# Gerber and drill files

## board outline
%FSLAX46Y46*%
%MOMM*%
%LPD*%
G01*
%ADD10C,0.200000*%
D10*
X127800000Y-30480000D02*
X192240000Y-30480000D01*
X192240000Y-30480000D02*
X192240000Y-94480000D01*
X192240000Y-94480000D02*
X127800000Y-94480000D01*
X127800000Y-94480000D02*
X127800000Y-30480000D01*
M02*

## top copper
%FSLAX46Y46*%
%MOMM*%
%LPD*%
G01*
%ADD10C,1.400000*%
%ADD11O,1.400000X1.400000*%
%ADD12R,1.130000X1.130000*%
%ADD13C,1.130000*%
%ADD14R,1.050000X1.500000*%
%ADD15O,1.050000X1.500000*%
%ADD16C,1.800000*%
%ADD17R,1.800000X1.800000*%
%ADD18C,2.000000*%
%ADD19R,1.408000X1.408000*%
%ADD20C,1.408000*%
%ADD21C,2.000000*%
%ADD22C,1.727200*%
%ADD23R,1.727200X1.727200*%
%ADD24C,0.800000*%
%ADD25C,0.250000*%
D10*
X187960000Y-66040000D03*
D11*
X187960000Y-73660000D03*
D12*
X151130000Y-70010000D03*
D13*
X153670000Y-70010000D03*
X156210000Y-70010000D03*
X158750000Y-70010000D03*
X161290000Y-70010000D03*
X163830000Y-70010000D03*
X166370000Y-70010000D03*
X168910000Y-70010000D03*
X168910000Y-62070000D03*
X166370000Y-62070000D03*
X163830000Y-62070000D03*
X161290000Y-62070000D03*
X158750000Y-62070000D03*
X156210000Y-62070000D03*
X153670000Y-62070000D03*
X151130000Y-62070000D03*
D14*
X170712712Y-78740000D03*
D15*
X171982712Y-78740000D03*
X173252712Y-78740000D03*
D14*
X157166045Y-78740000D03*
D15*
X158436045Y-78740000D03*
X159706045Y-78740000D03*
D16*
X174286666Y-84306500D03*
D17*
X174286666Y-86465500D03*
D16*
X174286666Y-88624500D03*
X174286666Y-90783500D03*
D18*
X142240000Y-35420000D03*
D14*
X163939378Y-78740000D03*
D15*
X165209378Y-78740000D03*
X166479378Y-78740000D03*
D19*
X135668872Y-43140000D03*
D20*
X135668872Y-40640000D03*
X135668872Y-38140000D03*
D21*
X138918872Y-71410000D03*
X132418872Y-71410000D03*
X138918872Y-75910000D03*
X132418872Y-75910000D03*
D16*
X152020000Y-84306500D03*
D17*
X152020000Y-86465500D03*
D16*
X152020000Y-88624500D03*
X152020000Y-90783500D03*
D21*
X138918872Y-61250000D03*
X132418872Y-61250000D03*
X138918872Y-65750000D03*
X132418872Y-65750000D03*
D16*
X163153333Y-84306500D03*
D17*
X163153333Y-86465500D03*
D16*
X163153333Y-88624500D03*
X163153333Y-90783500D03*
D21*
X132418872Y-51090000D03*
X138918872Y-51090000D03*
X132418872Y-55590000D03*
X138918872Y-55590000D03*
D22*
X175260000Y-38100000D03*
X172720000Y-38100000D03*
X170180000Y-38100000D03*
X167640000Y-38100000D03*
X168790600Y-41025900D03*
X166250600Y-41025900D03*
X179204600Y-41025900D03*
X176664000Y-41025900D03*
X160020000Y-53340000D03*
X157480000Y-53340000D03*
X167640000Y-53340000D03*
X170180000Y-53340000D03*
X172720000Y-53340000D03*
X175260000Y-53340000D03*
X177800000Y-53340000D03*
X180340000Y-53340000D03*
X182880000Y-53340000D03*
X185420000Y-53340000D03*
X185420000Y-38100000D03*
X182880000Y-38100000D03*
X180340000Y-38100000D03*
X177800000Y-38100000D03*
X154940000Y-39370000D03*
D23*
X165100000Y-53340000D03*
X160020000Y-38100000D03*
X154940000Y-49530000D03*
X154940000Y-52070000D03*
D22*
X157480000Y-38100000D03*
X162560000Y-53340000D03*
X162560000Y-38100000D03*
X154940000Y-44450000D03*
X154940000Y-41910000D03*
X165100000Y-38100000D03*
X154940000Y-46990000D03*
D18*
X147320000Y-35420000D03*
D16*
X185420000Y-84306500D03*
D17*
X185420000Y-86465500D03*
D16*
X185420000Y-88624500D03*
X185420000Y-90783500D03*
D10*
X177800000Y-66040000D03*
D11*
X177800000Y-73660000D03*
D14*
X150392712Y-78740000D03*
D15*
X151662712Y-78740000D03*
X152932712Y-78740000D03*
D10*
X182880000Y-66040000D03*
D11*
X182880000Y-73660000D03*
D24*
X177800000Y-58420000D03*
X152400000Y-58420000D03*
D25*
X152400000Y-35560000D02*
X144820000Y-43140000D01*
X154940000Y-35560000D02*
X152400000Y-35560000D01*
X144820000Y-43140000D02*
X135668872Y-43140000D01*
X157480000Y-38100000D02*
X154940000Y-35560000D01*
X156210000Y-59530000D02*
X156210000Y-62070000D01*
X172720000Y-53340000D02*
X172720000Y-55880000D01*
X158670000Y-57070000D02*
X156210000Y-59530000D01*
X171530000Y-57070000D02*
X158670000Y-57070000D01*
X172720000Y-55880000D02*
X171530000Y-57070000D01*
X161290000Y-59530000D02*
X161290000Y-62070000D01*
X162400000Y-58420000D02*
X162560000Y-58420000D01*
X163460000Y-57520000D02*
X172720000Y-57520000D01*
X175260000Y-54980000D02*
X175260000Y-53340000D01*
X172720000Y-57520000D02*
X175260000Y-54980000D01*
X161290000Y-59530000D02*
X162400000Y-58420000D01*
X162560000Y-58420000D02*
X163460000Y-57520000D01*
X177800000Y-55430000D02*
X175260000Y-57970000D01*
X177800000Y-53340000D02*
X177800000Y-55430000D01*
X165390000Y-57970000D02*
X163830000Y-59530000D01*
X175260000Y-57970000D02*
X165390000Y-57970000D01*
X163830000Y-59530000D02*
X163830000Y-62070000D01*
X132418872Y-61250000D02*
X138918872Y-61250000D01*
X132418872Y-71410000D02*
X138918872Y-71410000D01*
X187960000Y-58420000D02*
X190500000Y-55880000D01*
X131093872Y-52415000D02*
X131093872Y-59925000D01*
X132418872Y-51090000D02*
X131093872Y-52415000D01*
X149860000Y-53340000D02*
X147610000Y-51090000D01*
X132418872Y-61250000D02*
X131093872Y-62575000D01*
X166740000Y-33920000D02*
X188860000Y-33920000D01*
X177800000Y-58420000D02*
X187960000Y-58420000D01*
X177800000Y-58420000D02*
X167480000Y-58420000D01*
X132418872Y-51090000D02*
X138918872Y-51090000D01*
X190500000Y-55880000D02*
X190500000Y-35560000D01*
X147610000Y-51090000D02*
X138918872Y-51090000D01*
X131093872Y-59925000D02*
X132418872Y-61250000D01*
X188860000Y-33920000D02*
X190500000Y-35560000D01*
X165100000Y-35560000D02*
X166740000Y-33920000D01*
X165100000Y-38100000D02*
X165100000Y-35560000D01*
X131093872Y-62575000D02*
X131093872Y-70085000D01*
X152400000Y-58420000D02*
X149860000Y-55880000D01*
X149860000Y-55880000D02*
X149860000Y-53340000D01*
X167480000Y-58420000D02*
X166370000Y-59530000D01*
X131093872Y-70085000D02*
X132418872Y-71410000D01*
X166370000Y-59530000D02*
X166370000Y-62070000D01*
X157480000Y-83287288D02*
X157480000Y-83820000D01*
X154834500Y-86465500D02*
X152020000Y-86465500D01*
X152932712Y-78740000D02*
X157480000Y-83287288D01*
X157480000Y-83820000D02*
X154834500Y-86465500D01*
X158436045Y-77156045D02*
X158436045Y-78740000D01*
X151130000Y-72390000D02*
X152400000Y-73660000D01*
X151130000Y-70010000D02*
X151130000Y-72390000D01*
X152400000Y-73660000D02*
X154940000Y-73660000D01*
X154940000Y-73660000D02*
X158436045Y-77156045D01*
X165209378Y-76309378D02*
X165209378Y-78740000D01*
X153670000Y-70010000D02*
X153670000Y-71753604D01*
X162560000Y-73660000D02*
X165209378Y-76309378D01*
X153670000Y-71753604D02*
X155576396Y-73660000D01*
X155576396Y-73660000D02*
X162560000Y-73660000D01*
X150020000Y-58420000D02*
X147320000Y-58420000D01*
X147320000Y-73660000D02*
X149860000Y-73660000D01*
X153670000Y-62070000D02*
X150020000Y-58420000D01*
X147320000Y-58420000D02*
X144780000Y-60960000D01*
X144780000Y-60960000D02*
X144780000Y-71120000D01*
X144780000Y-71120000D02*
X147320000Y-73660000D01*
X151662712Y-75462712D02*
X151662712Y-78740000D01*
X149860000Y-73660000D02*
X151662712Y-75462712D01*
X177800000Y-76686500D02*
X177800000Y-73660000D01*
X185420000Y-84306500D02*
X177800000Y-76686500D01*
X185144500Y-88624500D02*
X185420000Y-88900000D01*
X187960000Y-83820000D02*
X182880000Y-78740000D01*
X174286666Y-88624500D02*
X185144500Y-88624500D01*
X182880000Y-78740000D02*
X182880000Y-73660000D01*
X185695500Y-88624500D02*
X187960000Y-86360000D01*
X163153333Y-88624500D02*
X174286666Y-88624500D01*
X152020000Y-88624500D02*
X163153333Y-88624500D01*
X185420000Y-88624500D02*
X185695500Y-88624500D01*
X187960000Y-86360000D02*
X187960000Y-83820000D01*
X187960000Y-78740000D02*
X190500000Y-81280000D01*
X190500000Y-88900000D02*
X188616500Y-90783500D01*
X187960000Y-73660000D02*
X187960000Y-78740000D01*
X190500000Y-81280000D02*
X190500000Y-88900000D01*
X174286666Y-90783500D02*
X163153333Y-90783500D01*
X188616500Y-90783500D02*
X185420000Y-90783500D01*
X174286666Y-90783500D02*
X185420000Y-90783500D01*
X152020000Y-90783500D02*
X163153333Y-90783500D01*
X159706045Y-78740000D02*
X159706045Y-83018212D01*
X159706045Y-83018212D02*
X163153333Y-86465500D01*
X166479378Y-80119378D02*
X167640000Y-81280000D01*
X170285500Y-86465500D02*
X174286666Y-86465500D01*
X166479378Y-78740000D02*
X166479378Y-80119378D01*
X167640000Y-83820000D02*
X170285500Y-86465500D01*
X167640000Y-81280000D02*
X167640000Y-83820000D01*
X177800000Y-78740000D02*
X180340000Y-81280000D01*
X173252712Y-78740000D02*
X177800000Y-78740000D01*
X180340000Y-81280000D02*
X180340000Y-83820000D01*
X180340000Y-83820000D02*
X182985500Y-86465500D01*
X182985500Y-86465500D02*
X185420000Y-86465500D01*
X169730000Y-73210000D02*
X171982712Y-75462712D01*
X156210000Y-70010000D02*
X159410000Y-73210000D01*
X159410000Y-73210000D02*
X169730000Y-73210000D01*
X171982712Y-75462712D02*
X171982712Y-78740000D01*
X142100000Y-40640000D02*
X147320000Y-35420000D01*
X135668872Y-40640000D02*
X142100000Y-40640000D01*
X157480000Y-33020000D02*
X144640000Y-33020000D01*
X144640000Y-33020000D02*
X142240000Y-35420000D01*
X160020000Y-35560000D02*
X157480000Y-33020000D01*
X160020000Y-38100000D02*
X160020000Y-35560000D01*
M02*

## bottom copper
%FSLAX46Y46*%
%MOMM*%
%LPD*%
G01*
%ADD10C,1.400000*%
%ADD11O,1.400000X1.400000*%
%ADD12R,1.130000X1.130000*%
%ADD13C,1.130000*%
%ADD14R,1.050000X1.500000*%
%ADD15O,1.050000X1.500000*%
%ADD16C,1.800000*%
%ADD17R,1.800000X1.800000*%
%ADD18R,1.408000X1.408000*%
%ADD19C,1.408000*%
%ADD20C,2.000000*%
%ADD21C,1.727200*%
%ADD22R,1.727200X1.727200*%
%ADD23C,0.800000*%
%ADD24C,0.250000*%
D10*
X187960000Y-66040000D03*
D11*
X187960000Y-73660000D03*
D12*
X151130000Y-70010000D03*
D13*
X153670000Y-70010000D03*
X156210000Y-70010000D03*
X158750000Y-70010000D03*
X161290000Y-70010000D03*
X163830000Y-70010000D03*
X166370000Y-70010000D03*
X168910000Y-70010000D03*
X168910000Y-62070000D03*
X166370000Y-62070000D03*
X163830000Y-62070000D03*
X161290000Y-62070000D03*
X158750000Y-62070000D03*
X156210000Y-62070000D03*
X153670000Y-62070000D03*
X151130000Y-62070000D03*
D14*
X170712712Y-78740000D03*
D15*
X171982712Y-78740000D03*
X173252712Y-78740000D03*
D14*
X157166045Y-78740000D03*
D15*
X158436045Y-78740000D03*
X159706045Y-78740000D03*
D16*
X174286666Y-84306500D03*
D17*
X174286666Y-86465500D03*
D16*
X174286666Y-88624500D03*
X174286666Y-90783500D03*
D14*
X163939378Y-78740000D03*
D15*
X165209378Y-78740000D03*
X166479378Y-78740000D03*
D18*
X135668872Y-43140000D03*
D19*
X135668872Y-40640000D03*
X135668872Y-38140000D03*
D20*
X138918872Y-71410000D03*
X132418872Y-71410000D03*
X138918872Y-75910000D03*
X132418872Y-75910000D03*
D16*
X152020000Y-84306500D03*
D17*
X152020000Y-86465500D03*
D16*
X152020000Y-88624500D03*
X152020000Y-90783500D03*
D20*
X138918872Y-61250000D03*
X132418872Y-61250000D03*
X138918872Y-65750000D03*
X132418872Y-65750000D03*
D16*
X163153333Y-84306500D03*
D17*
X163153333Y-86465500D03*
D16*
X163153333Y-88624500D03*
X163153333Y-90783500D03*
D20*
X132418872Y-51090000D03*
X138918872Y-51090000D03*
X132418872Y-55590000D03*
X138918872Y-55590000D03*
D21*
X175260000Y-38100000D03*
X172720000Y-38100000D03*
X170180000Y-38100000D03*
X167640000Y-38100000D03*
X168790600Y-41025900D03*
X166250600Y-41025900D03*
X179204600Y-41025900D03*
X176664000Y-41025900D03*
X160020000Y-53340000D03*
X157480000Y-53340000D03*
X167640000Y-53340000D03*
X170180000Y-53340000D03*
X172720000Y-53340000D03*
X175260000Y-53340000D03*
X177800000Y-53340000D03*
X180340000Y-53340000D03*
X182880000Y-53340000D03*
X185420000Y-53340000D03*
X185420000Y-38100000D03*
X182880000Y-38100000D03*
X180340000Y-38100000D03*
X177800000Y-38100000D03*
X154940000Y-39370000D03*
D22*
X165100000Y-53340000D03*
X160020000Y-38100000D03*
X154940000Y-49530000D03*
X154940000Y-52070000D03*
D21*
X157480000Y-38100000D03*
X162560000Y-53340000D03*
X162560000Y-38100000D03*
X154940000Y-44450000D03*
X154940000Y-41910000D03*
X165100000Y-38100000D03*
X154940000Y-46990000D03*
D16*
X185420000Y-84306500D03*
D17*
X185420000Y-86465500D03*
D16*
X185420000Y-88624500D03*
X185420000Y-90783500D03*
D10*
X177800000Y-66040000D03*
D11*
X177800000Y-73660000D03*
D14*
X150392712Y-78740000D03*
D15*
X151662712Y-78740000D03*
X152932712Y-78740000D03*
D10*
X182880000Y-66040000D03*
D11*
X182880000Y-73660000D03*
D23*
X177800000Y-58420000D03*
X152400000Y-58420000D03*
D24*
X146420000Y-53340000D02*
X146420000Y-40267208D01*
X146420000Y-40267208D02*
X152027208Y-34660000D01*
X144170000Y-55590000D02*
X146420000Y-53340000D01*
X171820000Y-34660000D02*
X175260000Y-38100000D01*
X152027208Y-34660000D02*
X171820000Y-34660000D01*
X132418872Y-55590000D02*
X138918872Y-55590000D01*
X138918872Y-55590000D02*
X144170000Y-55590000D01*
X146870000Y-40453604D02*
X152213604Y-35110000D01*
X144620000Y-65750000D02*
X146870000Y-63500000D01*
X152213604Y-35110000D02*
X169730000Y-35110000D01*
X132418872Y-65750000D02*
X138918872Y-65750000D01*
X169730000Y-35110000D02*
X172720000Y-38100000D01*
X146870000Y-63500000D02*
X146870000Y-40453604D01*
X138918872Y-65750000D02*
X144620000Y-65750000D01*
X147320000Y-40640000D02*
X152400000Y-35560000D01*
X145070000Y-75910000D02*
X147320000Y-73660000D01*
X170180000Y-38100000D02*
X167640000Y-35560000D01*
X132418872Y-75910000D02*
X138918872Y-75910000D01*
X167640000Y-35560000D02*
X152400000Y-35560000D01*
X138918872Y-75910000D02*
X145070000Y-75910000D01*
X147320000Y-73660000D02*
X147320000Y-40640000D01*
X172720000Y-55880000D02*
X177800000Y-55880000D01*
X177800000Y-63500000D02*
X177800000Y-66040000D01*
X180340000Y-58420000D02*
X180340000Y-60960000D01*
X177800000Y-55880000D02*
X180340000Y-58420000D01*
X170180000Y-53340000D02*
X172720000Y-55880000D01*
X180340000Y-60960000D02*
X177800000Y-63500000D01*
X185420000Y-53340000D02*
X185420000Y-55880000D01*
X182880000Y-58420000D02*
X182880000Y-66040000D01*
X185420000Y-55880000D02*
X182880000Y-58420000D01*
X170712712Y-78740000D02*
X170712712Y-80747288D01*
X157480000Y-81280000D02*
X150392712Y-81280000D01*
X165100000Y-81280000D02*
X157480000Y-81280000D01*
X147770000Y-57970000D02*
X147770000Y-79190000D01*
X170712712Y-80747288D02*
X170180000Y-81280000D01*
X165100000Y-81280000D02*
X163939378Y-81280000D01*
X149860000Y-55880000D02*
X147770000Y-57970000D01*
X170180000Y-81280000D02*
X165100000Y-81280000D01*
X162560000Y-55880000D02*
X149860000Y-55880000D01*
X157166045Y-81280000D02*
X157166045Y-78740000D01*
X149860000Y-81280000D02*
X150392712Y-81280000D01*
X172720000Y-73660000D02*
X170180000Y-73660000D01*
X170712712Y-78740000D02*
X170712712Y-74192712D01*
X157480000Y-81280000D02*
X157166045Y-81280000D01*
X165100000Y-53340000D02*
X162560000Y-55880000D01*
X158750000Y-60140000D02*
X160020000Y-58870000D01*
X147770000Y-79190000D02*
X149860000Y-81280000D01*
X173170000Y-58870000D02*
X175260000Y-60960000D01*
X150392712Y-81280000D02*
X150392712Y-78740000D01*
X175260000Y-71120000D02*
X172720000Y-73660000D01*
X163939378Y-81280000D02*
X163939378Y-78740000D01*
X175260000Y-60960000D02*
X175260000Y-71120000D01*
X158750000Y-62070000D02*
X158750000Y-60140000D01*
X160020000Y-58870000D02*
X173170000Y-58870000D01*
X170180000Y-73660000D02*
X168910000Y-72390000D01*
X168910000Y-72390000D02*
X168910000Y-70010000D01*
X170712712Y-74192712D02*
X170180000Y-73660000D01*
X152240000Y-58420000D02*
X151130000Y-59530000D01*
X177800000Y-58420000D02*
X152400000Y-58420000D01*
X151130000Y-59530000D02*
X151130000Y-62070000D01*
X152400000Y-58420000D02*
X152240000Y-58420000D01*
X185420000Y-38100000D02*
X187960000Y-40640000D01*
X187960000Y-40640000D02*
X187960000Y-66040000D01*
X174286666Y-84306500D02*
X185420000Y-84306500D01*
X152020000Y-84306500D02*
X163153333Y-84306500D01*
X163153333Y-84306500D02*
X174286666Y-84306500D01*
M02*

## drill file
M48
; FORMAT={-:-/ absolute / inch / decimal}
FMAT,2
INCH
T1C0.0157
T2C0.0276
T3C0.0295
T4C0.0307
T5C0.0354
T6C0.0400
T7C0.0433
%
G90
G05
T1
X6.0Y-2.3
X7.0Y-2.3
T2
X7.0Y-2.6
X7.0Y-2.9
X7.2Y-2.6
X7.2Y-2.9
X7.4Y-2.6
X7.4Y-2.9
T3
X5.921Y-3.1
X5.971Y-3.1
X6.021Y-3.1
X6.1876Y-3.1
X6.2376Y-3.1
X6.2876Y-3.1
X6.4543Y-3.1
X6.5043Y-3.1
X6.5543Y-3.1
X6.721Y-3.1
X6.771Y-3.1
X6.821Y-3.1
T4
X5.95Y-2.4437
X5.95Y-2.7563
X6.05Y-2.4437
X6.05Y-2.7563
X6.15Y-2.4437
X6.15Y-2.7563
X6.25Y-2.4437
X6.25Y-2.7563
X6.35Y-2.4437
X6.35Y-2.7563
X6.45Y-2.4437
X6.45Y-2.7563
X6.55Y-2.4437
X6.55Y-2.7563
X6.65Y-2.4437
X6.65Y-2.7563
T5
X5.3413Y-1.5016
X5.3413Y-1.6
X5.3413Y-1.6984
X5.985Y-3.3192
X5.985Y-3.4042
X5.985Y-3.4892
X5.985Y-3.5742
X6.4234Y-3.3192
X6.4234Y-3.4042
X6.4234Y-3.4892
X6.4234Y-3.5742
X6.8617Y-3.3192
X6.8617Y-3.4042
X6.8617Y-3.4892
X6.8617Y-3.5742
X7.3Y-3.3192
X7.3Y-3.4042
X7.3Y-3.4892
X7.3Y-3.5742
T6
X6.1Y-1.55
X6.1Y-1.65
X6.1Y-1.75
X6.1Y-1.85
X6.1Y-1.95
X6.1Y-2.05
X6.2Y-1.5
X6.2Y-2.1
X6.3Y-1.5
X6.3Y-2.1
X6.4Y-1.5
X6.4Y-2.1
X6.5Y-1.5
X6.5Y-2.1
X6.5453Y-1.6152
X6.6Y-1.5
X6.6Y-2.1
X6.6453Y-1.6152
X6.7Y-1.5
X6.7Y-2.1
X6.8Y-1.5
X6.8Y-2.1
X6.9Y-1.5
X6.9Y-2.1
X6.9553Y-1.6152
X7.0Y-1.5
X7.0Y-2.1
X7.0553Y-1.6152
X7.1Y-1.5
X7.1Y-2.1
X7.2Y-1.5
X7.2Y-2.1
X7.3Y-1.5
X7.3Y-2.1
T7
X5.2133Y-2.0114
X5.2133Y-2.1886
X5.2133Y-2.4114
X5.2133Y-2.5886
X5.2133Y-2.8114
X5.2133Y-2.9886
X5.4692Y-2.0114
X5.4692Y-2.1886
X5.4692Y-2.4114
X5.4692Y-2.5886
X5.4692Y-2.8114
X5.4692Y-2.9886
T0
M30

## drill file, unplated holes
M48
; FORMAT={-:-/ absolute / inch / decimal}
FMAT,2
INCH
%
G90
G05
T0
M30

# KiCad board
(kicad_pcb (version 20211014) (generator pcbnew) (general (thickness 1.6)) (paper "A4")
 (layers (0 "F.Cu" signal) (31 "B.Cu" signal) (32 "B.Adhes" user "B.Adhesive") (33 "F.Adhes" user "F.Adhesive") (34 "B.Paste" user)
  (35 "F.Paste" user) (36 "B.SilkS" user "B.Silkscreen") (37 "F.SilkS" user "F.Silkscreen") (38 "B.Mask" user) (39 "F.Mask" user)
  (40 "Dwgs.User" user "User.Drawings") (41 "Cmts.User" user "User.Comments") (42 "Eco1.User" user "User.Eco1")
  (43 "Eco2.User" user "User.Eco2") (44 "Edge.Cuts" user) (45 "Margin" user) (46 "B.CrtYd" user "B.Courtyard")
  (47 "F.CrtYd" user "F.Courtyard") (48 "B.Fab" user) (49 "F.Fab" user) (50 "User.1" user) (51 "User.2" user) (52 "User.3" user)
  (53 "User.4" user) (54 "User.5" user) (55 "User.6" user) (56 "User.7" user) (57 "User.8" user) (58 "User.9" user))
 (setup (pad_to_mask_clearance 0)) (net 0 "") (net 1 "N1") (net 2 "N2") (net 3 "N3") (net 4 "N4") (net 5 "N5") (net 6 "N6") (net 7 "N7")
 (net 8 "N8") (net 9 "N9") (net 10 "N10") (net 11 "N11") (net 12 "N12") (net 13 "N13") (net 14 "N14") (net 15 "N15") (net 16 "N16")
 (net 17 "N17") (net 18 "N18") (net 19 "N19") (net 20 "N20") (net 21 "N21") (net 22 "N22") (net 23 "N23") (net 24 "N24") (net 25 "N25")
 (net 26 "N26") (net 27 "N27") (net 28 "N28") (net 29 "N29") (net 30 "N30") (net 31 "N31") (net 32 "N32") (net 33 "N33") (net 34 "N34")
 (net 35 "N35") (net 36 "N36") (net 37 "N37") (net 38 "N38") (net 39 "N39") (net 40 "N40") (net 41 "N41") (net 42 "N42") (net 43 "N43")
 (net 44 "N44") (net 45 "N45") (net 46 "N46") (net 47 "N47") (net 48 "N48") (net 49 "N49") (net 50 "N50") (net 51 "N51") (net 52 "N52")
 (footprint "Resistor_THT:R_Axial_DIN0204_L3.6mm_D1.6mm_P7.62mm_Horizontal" (layer "F.Cu") (at 187.96 66.04 -90)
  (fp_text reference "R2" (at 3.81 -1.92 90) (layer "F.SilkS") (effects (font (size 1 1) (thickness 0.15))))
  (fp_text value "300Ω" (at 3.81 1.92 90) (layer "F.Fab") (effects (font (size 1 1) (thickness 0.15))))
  (pad "1" thru_hole circle (at 0 0 270) (size 1.4 1.4) (drill 0.7) (layers *.Cu *.Mask) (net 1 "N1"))
  (pad "2" thru_hole oval (at 7.62 0 270) (size 1.4 1.4) (drill 0.7) (layers *.Cu *.Mask) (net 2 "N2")))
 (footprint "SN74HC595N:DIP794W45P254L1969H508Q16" (layer "F.Cu") (at 160.02 66.04 90)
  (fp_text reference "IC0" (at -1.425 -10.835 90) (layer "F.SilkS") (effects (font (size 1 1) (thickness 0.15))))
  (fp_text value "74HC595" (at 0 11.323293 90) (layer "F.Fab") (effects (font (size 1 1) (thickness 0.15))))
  (pad "1" thru_hole rect locked (at -3.97 -8.89 90) (size 1.13 1.13) (drill 0.78) (layers *.Cu *.Mask) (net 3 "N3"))
  (pad "2" thru_hole circle locked (at -3.97 -6.35 90) (size 1.13 1.13) (drill 0.78) (layers *.Cu *.Mask) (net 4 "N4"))
  (pad "3" thru_hole circle locked (at -3.97 -3.81 90) (size 1.13 1.13) (drill 0.78) (layers *.Cu *.Mask) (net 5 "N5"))
  (pad "4" thru_hole circle locked (at -3.97 -1.27 90) (size 1.13 1.13) (drill 0.78) (layers *.Cu *.Mask) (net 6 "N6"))
  (pad "5" thru_hole circle locked (at -3.97 1.27 90) (size 1.13 1.13) (drill 0.78) (layers *.Cu *.Mask) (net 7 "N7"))
  (pad "6" thru_hole circle locked (at -3.97 3.81 90) (size 1.13 1.13) (drill 0.78) (layers *.Cu *.Mask) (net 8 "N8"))
  (pad "7" thru_hole circle locked (at -3.97 6.35 90) (size 1.13 1.13) (drill 0.78) (layers *.Cu *.Mask) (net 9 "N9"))
  (pad "8" thru_hole circle locked (at -3.97 8.89 90) (size 1.13 1.13) (drill 0.78) (layers *.Cu *.Mask) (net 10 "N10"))
  (pad "9" thru_hole circle locked (at 3.97 8.89 90) (size 1.13 1.13) (drill 0.78) (layers *.Cu *.Mask) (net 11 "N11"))
  (pad "10" thru_hole circle locked (at 3.97 6.35 90) (size 1.13 1.13) (drill 0.78) (layers *.Cu *.Mask) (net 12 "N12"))
  (pad "11" thru_hole circle locked (at 3.97 3.81 90) (size 1.13 1.13) (drill 0.78) (layers *.Cu *.Mask) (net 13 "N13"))
  (pad "12" thru_hole circle locked (at 3.97 1.27 90) (size 1.13 1.13) (drill 0.78) (layers *.Cu *.Mask) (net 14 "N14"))
  (pad "13" thru_hole circle locked (at 3.97 -1.27 90) (size 1.13 1.13) (drill 0.78) (layers *.Cu *.Mask) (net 10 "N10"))
  (pad "14" thru_hole circle locked (at 3.97 -3.81 90) (size 1.13 1.13) (drill 0.78) (layers *.Cu *.Mask) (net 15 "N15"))
  (pad "15" thru_hole circle locked (at 3.97 -6.35 90) (size 1.13 1.13) (drill 0.78) (layers *.Cu *.Mask) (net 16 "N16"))
  (pad "16" thru_hole circle locked (at 3.97 -8.89 90) (size 1.13 1.13) (drill 0.78) (layers *.Cu *.Mask) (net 12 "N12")))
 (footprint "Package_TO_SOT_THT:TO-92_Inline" (layer "F.Cu") (at 170.712712 78.74)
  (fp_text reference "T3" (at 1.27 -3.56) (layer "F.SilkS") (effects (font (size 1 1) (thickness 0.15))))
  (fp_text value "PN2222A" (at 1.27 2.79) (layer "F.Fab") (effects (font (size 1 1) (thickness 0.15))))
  (pad "1" thru_hole rect (at 0 0) (size 1.05 1.5) (drill 0.75) (layers *.Cu *.Mask) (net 10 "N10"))
  (pad "2" thru_hole oval (at 1.27 0) (size 1.05 1.5) (drill 0.75) (layers *.Cu *.Mask) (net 5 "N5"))
  (pad "3" thru_hole oval (at 2.54 0) (size 1.05 1.5) (drill 0.75) (layers *.Cu *.Mask) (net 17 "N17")))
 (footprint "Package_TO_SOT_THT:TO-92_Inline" (layer "F.Cu") (at 157.166045 78.74)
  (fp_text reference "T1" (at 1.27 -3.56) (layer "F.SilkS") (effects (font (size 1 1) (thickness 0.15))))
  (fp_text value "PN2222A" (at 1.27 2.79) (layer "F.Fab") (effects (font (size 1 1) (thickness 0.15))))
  (pad "1" thru_hole rect (at 0 0) (size 1.05 1.5) (drill 0.75) (layers *.Cu *.Mask) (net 10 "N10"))
  (pad "2" thru_hole oval (at 1.27 0) (size 1.05 1.5) (drill 0.75) (layers *.Cu *.Mask) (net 3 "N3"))
  (pad "3" thru_hole oval (at 2.54 0) (size 1.05 1.5) (drill 0.75) (layers *.Cu *.Mask) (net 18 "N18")))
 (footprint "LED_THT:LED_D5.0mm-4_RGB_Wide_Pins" (layer "F.Cu") (at 174.286666 84.3065 -90)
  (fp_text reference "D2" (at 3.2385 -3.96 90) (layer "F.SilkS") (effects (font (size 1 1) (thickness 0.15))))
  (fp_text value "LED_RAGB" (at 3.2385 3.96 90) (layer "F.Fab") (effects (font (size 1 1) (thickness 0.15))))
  (pad "1" thru_hole circle (at 0 0 270) (size 1.8 1.8) (drill 0.9) (layers *.Cu *.Mask) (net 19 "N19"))
  (pad "2" thru_hole rect (at 2.159 0 270) (size 1.8 1.8) (drill 0.9) (layers *.Cu *.Mask) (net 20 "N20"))
  (pad "3" thru_hole circle (at 4.318 0 270) (size 1.8 1.8) (drill 0.9) (layers *.Cu *.Mask) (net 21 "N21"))
  (pad "4" thru_hole circle (at 6.477 0 270) (size 1.8 1.8) (drill 0.9) (layers *.Cu *.Mask) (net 2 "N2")))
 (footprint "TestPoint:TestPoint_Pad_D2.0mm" (layer "F.Cu") (at 142.24 35.42)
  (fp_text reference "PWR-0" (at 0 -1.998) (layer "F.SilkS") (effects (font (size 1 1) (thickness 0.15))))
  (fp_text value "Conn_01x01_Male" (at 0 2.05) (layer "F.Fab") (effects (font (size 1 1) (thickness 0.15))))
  (pad "1" smd circle (at 0 0) (size 2 2) (layers "F.Cu" "F.Mask") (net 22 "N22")))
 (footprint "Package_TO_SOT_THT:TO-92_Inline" (layer "F.Cu") (at 163.939378 78.74)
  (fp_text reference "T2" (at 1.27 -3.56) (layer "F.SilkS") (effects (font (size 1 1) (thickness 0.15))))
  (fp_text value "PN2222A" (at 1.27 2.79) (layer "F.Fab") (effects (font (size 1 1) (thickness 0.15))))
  (pad "1" thru_hole rect (at 0 0) (size 1.05 1.5) (drill 0.75) (layers *.Cu *.Mask) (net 10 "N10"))
  (pad "2" thru_hole oval (at 1.27 0) (size 1.05 1.5) (drill 0.75) (layers *.Cu *.Mask) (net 4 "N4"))
  (pad "3" thru_hole oval (at 2.54 0) (size 1.05 1.5) (drill 0.75) (layers *.Cu *.Mask) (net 20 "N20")))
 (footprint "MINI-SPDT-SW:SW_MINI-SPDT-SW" (layer "F.Cu") (at 135.668872 40.64 90)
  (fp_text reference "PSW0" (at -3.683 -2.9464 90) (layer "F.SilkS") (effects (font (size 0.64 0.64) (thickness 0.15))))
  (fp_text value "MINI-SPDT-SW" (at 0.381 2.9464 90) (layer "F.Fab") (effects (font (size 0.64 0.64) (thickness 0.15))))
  (pad "1" thru_hole rect locked (at -2.5 0 90) (size 1.408 1.408) (drill 0.9) (layers *.Cu *.Mask) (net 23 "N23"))
  (pad "2" thru_hole circle locked (at 0 0 90) (size 1.408 1.408) (drill 0.9) (layers *.Cu *.Mask) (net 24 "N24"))
  (pad "3" thru_hole circle locked (at 2.5 0 90) (size 1.408 1.408) (drill 0.9) (layers *.Cu *.Mask) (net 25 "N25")))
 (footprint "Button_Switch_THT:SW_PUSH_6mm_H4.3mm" (layer "F.Cu") (at 132.418872 71.41)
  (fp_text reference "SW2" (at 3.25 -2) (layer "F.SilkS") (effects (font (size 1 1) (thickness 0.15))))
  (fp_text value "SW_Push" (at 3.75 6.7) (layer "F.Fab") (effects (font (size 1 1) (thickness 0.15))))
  (pad "1" thru_hole circle (at 6.5 0 90) (size 2 2) (drill 1.1) (layers *.Cu *.Mask) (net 12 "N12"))
  (pad "1" thru_hole circle (at 0 0 90) (size 2 2) (drill 1.1) (layers *.Cu *.Mask) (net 12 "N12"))
  (pad "2" thru_hole circle (at 6.5 4.5 90) (size 2 2) (drill 1.1) (layers *.Cu *.Mask) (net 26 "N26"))
  (pad "2" thru_hole circle (at 0 4.5 90) (size 2 2) (drill 1.1) (layers *.Cu *.Mask) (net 26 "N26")))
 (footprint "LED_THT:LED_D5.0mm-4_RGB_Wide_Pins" (layer "F.Cu") (at 152.02 84.3065 -90)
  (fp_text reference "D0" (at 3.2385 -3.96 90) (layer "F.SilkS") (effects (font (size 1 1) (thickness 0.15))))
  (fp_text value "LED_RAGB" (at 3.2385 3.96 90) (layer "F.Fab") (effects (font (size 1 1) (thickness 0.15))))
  (pad "1" thru_hole circle (at 0 0 270) (size 1.8 1.8) (drill 0.9) (layers *.Cu *.Mask) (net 19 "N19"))
  (pad "2" thru_hole rect (at 2.159 0 270) (size 1.8 1.8) (drill 0.9) (layers *.Cu *.Mask) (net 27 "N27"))
  (pad "3" thru_hole circle (at 4.318 0 270) (size 1.8 1.8) (drill 0.9) (layers *.Cu *.Mask) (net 21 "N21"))
  (pad "4" thru_hole circle (at 6.477 0 270) (size 1.8 1.8) (drill 0.9) (layers *.Cu *.Mask) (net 2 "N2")))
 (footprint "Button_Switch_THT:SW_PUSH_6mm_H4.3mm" (layer "F.Cu") (at 132.418872 61.25)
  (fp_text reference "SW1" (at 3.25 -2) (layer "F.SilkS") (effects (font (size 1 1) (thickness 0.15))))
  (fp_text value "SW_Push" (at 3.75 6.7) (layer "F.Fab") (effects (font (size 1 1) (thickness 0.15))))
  (pad "1" thru_hole circle (at 6.5 0 90) (size 2 2) (drill 1.1) (layers *.Cu *.Mask) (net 12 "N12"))
  (pad "1" thru_hole circle (at 0 0 90) (size 2 2) (drill 1.1) (layers *.Cu *.Mask) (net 12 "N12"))
  (pad "2" thru_hole circle (at 6.5 4.5 90) (size 2 2) (drill 1.1) (layers *.Cu *.Mask) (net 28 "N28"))
  (pad "2" thru_hole circle (at 0 4.5 90) (size 2 2) (drill 1.1) (layers *.Cu *.Mask) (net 28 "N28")))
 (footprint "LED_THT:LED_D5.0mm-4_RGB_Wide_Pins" (layer "F.Cu") (at 163.153333 84.3065 -90)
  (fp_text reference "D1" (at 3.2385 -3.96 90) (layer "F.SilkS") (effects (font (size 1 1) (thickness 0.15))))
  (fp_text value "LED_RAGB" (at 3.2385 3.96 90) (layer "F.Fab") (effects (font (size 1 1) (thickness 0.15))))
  (pad "1" thru_hole circle (at 0 0 270) (size 1.8 1.8) (drill 0.9) (layers *.Cu *.Mask) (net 19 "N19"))
  (pad "2" thru_hole rect (at 2.159 0 270) (size 1.8 1.8) (drill 0.9) (layers *.Cu *.Mask) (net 18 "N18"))
  (pad "3" thru_hole circle (at 4.318 0 270) (size 1.8 1.8) (drill 0.9) (layers *.Cu *.Mask) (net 21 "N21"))
  (pad "4" thru_hole circle (at 6.477 0 270) (size 1.8 1.8) (drill 0.9) (layers *.Cu *.Mask) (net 2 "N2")))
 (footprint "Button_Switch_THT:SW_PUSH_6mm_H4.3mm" (layer "F.Cu") (at 132.418872 51.09)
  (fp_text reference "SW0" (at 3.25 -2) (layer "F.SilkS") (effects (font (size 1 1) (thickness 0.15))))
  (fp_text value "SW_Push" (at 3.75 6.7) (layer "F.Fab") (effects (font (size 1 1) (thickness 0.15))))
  (pad "1" thru_hole circle (at 0 0 90) (size 2 2) (drill 1.1) (layers *.Cu *.Mask) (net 12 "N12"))
  (pad "1" thru_hole circle (at 6.5 0 90) (size 2 2) (drill 1.1) (layers *.Cu *.Mask) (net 12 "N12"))
  (pad "2" thru_hole circle (at 0 4.5 90) (size 2 2) (drill 1.1) (layers *.Cu *.Mask) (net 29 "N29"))
  (pad "2" thru_hole circle (at 6.5 4.5 90) (size 2 2) (drill 1.1) (layers *.Cu *.Mask) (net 29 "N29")))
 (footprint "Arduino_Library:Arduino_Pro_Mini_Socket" (layer "F.Cu") (at 170.18 45.72 90)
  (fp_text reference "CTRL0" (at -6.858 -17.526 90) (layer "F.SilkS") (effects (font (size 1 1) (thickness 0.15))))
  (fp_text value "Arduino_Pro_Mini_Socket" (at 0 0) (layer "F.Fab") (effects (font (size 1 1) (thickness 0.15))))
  (pad "A0" thru_hole circle (at 7.62 5.08 90) (size 1.7272 1.7272) (drill 1.016) (layers *.Cu *.Mask) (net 29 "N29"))
  (pad "A1" thru_hole circle (at 7.62 2.54 90) (size 1.7272 1.7272) (drill 1.016) (layers *.Cu *.Mask) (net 28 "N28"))
  (pad "A2" thru_hole circle (at 7.62 0 90) (size 1.7272 1.7272) (drill 1.016) (layers *.Cu *.Mask) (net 26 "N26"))
  (pad "A3" thru_hole circle (at 7.62 -2.54 90) (size 1.7272 1.7272) (drill 1.016) (layers *.Cu *.Mask) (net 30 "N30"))
  (pad "A4" thru_hole circle (at 4.6941 -1.3894 90) (size 1.7272 1.7272) (drill 1.016) (layers *.Cu *.Mask) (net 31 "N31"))
  (pad "A5" thru_hole circle (at 4.6941 -3.9294 90) (size 1.7272 1.7272) (drill 1.016) (layers *.Cu *.Mask) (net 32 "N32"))
  (pad "A6" thru_hole circle (at 4.6941 9.0246 90) (size 1.7272 1.7272) (drill 1.016) (layers *.Cu *.Mask) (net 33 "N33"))
  (pad "A7" thru_hole circle (at 4.6941 6.484 90) (size 1.7272 1.7272) (drill 1.016) (layers *.Cu *.Mask) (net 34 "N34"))
  (pad "D0" thru_hole circle (at -7.62 -10.16 90) (size 1.7272 1.7272) (drill 1.016) (layers *.Cu *.Mask) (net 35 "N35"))
  (pad "D1" thru_hole circle (at -7.62 -12.7 90) (size 1.7272 1.7272) (drill 1.016) (layers *.Cu *.Mask) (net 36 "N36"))
  (pad "D2" thru_hole circle (at -7.62 -2.54 90) (size 1.7272 1.7272) (drill 1.016) (layers *.Cu *.Mask) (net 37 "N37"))
  (pad "D3" thru_hole circle (at -7.62 0 90) (size 1.7272 1.7272) (drill 1.016) (layers *.Cu *.Mask) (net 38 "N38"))
  (pad "D4" thru_hole circle (at -7.62 2.54 90) (size 1.7272 1.7272) (drill 1.016) (layers *.Cu *.Mask) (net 15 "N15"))
  (pad "D5" thru_hole circle (at -7.62 5.08 90) (size 1.7272 1.7272) (drill 1.016) (layers *.Cu *.Mask) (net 14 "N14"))
  (pad "D6" thru_hole circle (at -7.62 7.62 90) (size 1.7272 1.7272) (drill 1.016) (layers *.Cu *.Mask) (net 13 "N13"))
  (pad "D7" thru_hole circle (at -7.62 10.16 90) (size 1.7272 1.7272) (drill 1.016) (layers *.Cu *.Mask) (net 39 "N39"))
  (pad "D8" thru_hole circle (at -7.62 12.7 90) (size 1.7272 1.7272) (drill 1.016) (layers *.Cu *.Mask) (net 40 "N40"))
  (pad "D9" thru_hole circle (at -7.62 15.24 90) (size 1.7272 1.7272) (drill 1.016) (layers *.Cu *.Mask) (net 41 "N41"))
  (pad "D10" thru_hole circle (at 7.62 15.24 90) (size 1.7272 1.7272) (drill 1.016) (layers *.Cu *.Mask) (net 1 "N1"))
  (pad "D11" thru_hole circle (at 7.62 12.7 90) (size 1.7272 1.7272) (drill 1.016) (layers *.Cu *.Mask) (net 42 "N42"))
  (pad "D12" thru_hole circle (at 7.62 10.16 90) (size 1.7272 1.7272) (drill 1.016) (layers *.Cu *.Mask) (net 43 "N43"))
  (pad "D13" thru_hole circle (at 7.62 7.62 90) (size 1.7272 1.7272) (drill 1.016) (layers *.Cu *.Mask) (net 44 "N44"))
  (pad "DTR" thru_hole circle (at 6.35 -15.24 90) (size 1.7272 1.7272) (drill 1.016) (layers *.Cu *.Mask) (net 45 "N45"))
  (pad "GND1" thru_hole rect (at -7.62 -5.08 90) (size 1.7272 1.7272) (drill 1.016) (layers *.Cu *.Mask) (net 10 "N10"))
  (pad "GND2" thru_hole rect (at 7.62 -10.16 90) (size 1.7272 1.7272) (drill 1.016) (layers *.Cu *.Mask) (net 22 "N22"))
  (pad "GND4" thru_hole rect (at -3.81 -15.24 90) (size 1.7272 1.7272) (drill 1.016) (layers *.Cu *.Mask) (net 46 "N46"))
  (pad "GND5" thru_hole rect (at -6.35 -15.24 90) (size 1.7272 1.7272) (drill 1.016) (layers *.Cu *.Mask) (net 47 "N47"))
  (pad "RAW" thru_hole circle (at 7.62 -12.7 90) (size 1.7272 1.7272) (drill 1.016) (layers *.Cu *.Mask) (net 23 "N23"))
  (pad "RST1" thru_hole circle (at -7.62 -7.62 90) (size 1.7272 1.7272) (drill 1.016) (layers *.Cu *.Mask) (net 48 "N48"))
  (pad "RST2" thru_hole circle (at 7.62 -7.62 90) (size 1.7272 1.7272) (drill 1.016) (layers *.Cu *.Mask) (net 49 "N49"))
  (pad "RXI" thru_hole circle (at 1.27 -15.24 90) (size 1.7272 1.7272) (drill 1.016) (layers *.Cu *.Mask) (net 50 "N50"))
  (pad "TXO" thru_hole circle (at 3.81 -15.24 90) (size 1.7272 1.7272) (drill 1.016) (layers *.Cu *.Mask) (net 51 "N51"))
  (pad "Vcc1" thru_hole circle (at 7.62 -5.08 90) (size 1.7272 1.7272) (drill 1.016) (layers *.Cu *.Mask) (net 12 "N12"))
  (pad "Vcc2" thru_hole circle (at -1.27 -15.24 90) (size 1.7272 1.7272) (drill 1.016) (layers *.Cu *.Mask) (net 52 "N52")))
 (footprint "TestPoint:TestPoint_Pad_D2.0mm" (layer "F.Cu") (at 147.32 35.42)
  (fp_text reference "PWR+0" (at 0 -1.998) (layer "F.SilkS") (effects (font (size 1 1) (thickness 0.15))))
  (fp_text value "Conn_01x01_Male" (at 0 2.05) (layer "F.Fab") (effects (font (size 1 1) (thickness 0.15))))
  (pad "1" smd circle (at 0 0) (size 2 2) (layers "F.Cu" "F.Mask") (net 24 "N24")))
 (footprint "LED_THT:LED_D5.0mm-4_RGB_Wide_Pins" (layer "F.Cu") (at 185.42 84.3065 -90)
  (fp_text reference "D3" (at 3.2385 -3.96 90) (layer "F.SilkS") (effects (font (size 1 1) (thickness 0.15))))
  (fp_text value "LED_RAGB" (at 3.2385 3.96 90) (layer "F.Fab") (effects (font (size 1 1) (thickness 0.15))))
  (pad "1" thru_hole circle (at 0 0 270) (size 1.8 1.8) (drill 0.9) (layers *.Cu *.Mask) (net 19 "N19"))
  (pad "2" thru_hole rect (at 2.159 0 270) (size 1.8 1.8) (drill 0.9) (layers *.Cu *.Mask) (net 17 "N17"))
  (pad "3" thru_hole circle (at 4.318 0 270) (size 1.8 1.8) (drill 0.9) (layers *.Cu *.Mask) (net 21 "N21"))
  (pad "4" thru_hole circle (at 6.477 0 270) (size 1.8 1.8) (drill 0.9) (layers *.Cu *.Mask) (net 2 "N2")))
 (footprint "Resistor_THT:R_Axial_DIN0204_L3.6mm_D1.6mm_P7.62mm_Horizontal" (layer "F.Cu") (at 177.8 66.04 -90)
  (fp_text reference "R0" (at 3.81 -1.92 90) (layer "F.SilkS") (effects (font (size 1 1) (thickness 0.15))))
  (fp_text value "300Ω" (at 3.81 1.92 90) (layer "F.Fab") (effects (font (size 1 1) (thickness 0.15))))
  (pad "1" thru_hole circle (at 0 0 270) (size 1.4 1.4) (drill 0.7) (layers *.Cu *.Mask) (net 38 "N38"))
  (pad "2" thru_hole oval (at 7.62 0 270) (size 1.4 1.4) (drill 0.7) (layers *.Cu *.Mask) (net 19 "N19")))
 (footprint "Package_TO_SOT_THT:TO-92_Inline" (layer "F.Cu") (at 150.392712 78.74)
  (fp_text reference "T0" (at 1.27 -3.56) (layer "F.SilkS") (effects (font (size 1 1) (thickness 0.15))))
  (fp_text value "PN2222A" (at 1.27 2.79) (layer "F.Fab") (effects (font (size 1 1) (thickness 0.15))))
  (pad "1" thru_hole rect (at 0 0) (size 1.05 1.5) (drill 0.75) (layers *.Cu *.Mask) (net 10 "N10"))
  (pad "2" thru_hole oval (at 1.27 0) (size 1.05 1.5) (drill 0.75) (layers *.Cu *.Mask) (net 16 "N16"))
  (pad "3" thru_hole oval (at 2.54 0) (size 1.05 1.5) (drill 0.75) (layers *.Cu *.Mask) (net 27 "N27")))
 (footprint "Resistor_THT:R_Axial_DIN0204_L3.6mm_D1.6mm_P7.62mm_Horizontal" (layer "F.Cu") (at 182.88 66.04 -90)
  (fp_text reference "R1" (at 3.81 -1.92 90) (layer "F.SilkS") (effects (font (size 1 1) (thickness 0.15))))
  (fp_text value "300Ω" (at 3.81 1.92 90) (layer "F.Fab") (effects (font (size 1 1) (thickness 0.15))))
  (pad "1" thru_hole circle (at 0 0 270) (size 1.4 1.4) (drill 0.7) (layers *.Cu *.Mask) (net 41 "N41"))
  (pad "2" thru_hole oval (at 7.62 0 270) (size 1.4 1.4) (drill 0.7) (layers *.Cu *.Mask) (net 21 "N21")))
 (gr_rect (start 127.8 30.48) (end 192.24 94.48) (layer "Edge.Cuts") (width 0.2) (fill none))
 (segment (start 152.4 35.56) (end 144.82 43.14) (width 0.25) (layer "F.Cu") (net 23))
 (segment (start 154.94 35.56) (end 152.4 35.56) (width 0.25) (layer "F.Cu") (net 23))
 (segment (start 144.82 43.14) (end 135.668872 43.14) (width 0.25) (layer "F.Cu") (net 23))
 (segment (start 157.48 38.1) (end 154.94 35.56) (width 0.25) (layer "F.Cu") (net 23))
 (segment (start 146.42 53.34) (end 146.42 40.267208) (width 0.25) (layer "B.Cu") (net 29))
 (segment (start 146.42 40.267208) (end 152.027208 34.66) (width 0.25) (layer "B.Cu") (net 29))
 (segment (start 144.17 55.59) (end 146.42 53.34) (width 0.25) (layer "B.Cu") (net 29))
 (segment (start 171.82 34.66) (end 175.26 38.1) (width 0.25) (layer "B.Cu") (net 29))
 (segment (start 152.027208 34.66) (end 171.82 34.66) (width 0.25) (layer "B.Cu") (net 29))
 (segment (start 132.418872 55.59) (end 138.918872 55.59) (width 0.25) (layer "B.Cu") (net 29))
 (segment (start 138.918872 55.59) (end 144.17 55.59) (width 0.25) (layer "B.Cu") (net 29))
 (segment (start 146.87 40.453604) (end 152.213604 35.11) (width 0.25) (layer "B.Cu") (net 28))
 (segment (start 144.62 65.75) (end 146.87 63.5) (width 0.25) (layer "B.Cu") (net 28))
 (segment (start 152.213604 35.11) (end 169.73 35.11) (width 0.25) (layer "B.Cu") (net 28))
 (segment (start 132.418872 65.75) (end 138.918872 65.75) (width 0.25) (layer "B.Cu") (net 28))
 (segment (start 169.73 35.11) (end 172.72 38.1) (width 0.25) (layer "B.Cu") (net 28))
 (segment (start 146.87 63.5) (end 146.87 40.453604) (width 0.25) (layer "B.Cu") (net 28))
 (segment (start 138.918872 65.75) (end 144.62 65.75) (width 0.25) (layer "B.Cu") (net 28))
 (segment (start 147.32 40.64) (end 152.4 35.56) (width 0.25) (layer "B.Cu") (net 26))
 (segment (start 145.07 75.91) (end 147.32 73.66) (width 0.25) (layer "B.Cu") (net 26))
 (segment (start 170.18 38.1) (end 167.64 35.56) (width 0.25) (layer "B.Cu") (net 26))
 (segment (start 132.418872 75.91) (end 138.918872 75.91) (width 0.25) (layer "B.Cu") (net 26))
 (segment (start 167.64 35.56) (end 152.4 35.56) (width 0.25) (layer "B.Cu") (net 26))
 (segment (start 138.918872 75.91) (end 145.07 75.91) (width 0.25) (layer "B.Cu") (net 26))
 (segment (start 147.32 73.66) (end 147.32 40.64) (width 0.25) (layer "B.Cu") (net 26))
 (segment (start 156.21 59.53) (end 156.21 62.07) (width 0.25) (layer "F.Cu") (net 15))
 (segment (start 172.72 53.34) (end 172.72 55.88) (width 0.25) (layer "F.Cu") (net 15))
 (segment (start 158.67 57.07) (end 156.21 59.53) (width 0.25) (layer "F.Cu") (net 15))
 (segment (start 171.53 57.07) (end 158.67 57.07) (width 0.25) (layer "F.Cu") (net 15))
 (segment (start 172.72 55.88) (end 171.53 57.07) (width 0.25) (layer "F.Cu") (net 15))
 (segment (start 161.29 59.53) (end 161.29 62.07) (width 0.25) (layer "F.Cu") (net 14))
 (segment (start 162.4 58.42) (end 162.56 58.42) (width 0.25) (layer "F.Cu") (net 14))
 (segment (start 163.46 57.52) (end 172.72 57.52) (width 0.25) (layer "F.Cu") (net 14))
 (segment (start 175.26 54.98) (end 175.26 53.34) (width 0.25) (layer "F.Cu") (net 14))
 (segment (start 172.72 57.52) (end 175.26 54.98) (width 0.25) (layer "F.Cu") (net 14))
 (segment (start 161.29 59.53) (end 162.4 58.42) (width 0.25) (layer "F.Cu") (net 14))
 (segment (start 162.56 58.42) (end 163.46 57.52) (width 0.25) (layer "F.Cu") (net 14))
 (segment (start 177.8 55.43) (end 175.26 57.97) (width 0.25) (layer "F.Cu") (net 13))
 (segment (start 177.8 53.34) (end 177.8 55.43) (width 0.25) (layer "F.Cu") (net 13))
 (segment (start 165.39 57.97) (end 163.83 59.53) (width 0.25) (layer "F.Cu") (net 13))
 (segment (start 175.26 57.97) (end 165.39 57.97) (width 0.25) (layer "F.Cu") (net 13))
 (segment (start 163.83 59.53) (end 163.83 62.07) (width 0.25) (layer "F.Cu") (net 13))
 (segment (start 172.72 55.88) (end 177.8 55.88) (width 0.25) (layer "B.Cu") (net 38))
 (segment (start 177.8 63.5) (end 177.8 66.04) (width 0.25) (layer "B.Cu") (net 38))
 (segment (start 180.34 58.42) (end 180.34 60.96) (width 0.25) (layer "B.Cu") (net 38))
 (segment (start 177.8 55.88) (end 180.34 58.42) (width 0.25) (layer "B.Cu") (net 38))
 (segment (start 170.18 53.34) (end 172.72 55.88) (width 0.25) (layer "B.Cu") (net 38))
 (segment (start 180.34 60.96) (end 177.8 63.5) (width 0.25) (layer "B.Cu") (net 38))
 (segment (start 185.42 53.34) (end 185.42 55.88) (width 0.25) (layer "B.Cu") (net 41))
 (segment (start 182.88 58.42) (end 182.88 66.04) (width 0.25) (layer "B.Cu") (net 41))
 (segment (start 185.42 55.88) (end 182.88 58.42) (width 0.25) (layer "B.Cu") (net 41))
 (segment (start 170.712712 78.74) (end 170.712712 80.747288) (width 0.25) (layer "B.Cu") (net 10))
 (segment (start 157.48 81.28) (end 150.392712 81.28) (width 0.25) (layer "B.Cu") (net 10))
 (segment (start 165.1 81.28) (end 157.48 81.28) (width 0.25) (layer "B.Cu") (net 10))
 (segment (start 147.77 57.97) (end 147.77 79.19) (width 0.25) (layer "B.Cu") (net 10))
 (segment (start 170.712712 80.747288) (end 170.18 81.28) (width 0.25) (layer "B.Cu") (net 10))
 (segment (start 165.1 81.28) (end 163.939378 81.28) (width 0.25) (layer "B.Cu") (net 10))
 (segment (start 149.86 55.88) (end 147.77 57.97) (width 0.25) (layer "B.Cu") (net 10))
 (segment (start 170.18 81.28) (end 165.1 81.28) (width 0.25) (layer "B.Cu") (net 10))
 (segment (start 162.56 55.88) (end 149.86 55.88) (width 0.25) (layer "B.Cu") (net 10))
 (segment (start 157.166045 81.28) (end 157.166045 78.74) (width 0.25) (layer "B.Cu") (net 10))
 (segment (start 149.86 81.28) (end 150.392712 81.28) (width 0.25) (layer "B.Cu") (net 10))
 (segment (start 172.72 73.66) (end 170.18 73.66) (width 0.25) (layer "B.Cu") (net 10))
 (segment (start 170.712712 78.74) (end 170.712712 74.192712) (width 0.25) (layer "B.Cu") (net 10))
 (segment (start 157.48 81.28) (end 157.166045 81.28) (width 0.25) (layer "B.Cu") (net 10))
 (segment (start 165.1 53.34) (end 162.56 55.88) (width 0.25) (layer "B.Cu") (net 10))
 (segment (start 158.75 60.14) (end 160.02 58.87) (width 0.25) (layer "B.Cu") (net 10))
 (segment (start 147.77 79.19) (end 149.86 81.28) (width 0.25) (layer "B.Cu") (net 10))
 (segment (start 173.17 58.87) (end 175.26 60.96) (width 0.25) (layer "B.Cu") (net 10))
 (segment (start 150.392712 81.28) (end 150.392712 78.74) (width 0.25) (layer "B.Cu") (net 10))
 (segment (start 175.26 71.12) (end 172.72 73.66) (width 0.25) (layer "B.Cu") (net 10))
 (segment (start 163.939378 81.28) (end 163.939378 78.74) (width 0.25) (layer "B.Cu") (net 10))
 (segment (start 175.26 60.96) (end 175.26 71.12) (width 0.25) (layer "B.Cu") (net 10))
 (segment (start 158.75 62.07) (end 158.75 60.14) (width 0.25) (layer "B.Cu") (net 10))
 (segment (start 160.02 58.87) (end 173.17 58.87) (width 0.25) (layer "B.Cu") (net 10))
 (segment (start 170.18 73.66) (end 168.91 72.39) (width 0.25) (layer "B.Cu") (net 10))
 (segment (start 168.91 72.39) (end 168.91 70.01) (width 0.25) (layer "B.Cu") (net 10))
 (segment (start 170.712712 74.192712) (end 170.18 73.66) (width 0.25) (layer "B.Cu") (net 10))
 (segment (start 132.418872 61.25) (end 138.918872 61.25) (width 0.25) (layer "F.Cu") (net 12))
 (segment (start 132.418872 71.41) (end 138.918872 71.41) (width 0.25) (layer "F.Cu") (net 12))
 (segment (start 187.96 58.42) (end 190.5 55.88) (width 0.25) (layer "F.Cu") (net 12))
 (segment (start 131.093872 52.415) (end 131.093872 59.925) (width 0.25) (layer "F.Cu") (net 12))
 (segment (start 132.418872 51.09) (end 131.093872 52.415) (width 0.25) (layer "F.Cu") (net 12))
 (segment (start 149.86 53.34) (end 147.61 51.09) (width 0.25) (layer "F.Cu") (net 12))
 (segment (start 132.418872 61.25) (end 131.093872 62.575) (width 0.25) (layer "F.Cu") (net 12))
 (segment (start 166.74 33.92) (end 188.86 33.92) (width 0.25) (layer "F.Cu") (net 12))
 (segment (start 177.8 58.42) (end 187.96 58.42) (width 0.25) (layer "F.Cu") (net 12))
 (segment (start 177.8 58.42) (end 167.48 58.42) (width 0.25) (layer "F.Cu") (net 12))
 (segment (start 132.418872 51.09) (end 138.918872 51.09) (width 0.25) (layer "F.Cu") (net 12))
 (segment (start 190.5 55.88) (end 190.5 35.56) (width 0.25) (layer "F.Cu") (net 12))
 (segment (start 147.61 51.09) (end 138.918872 51.09) (width 0.25) (layer "F.Cu") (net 12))
 (segment (start 131.093872 59.925) (end 132.418872 61.25) (width 0.25) (layer "F.Cu") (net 12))
 (segment (start 188.86 33.92) (end 190.5 35.56) (width 0.25) (layer "F.Cu") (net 12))
 (segment (start 165.1 35.56) (end 166.74 33.92) (width 0.25) (layer "F.Cu") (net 12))
 (segment (start 165.1 38.1) (end 165.1 35.56) (width 0.25) (layer "F.Cu") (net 12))
 (segment (start 131.093872 62.575) (end 131.093872 70.085) (width 0.25) (layer "F.Cu") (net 12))
 (segment (start 152.4 58.42) (end 149.86 55.88) (width 0.25) (layer "F.Cu") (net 12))
 (segment (start 149.86 55.88) (end 149.86 53.34) (width 0.25) (layer "F.Cu") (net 12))
 (segment (start 167.48 58.42) (end 166.37 59.53) (width 0.25) (layer "F.Cu") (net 12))
 (segment (start 131.093872 70.085) (end 132.418872 71.41) (width 0.25) (layer "F.Cu") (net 12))
 (segment (start 166.37 59.53) (end 166.37 62.07) (width 0.25) (layer "F.Cu") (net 12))
 (via (at 177.8 58.42) (size 0.8) (drill 0.4) (layers "F.Cu" "B.Cu") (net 12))
 (via (at 152.4 58.42) (size 0.8) (drill 0.4) (layers "F.Cu" "B.Cu") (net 12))
 (segment (start 152.24 58.42) (end 151.13 59.53) (width 0.25) (layer "B.Cu") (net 12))
 (segment (start 177.8 58.42) (end 152.4 58.42) (width 0.25) (layer "B.Cu") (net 12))
 (segment (start 151.13 59.53) (end 151.13 62.07) (width 0.25) (layer "B.Cu") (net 12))
 (segment (start 152.4 58.42) (end 152.24 58.42) (width 0.25) (layer "B.Cu") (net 12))
 (segment (start 157.48 83.287288) (end 157.48 83.82) (width 0.25) (layer "F.Cu") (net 27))
 (segment (start 154.8345 86.4655) (end 152.02 86.4655) (width 0.25) (layer "F.Cu") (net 27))
 (segment (start 152.932712 78.74) (end 157.48 83.287288) (width 0.25) (layer "F.Cu") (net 27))
 (segment (start 157.48 83.82) (end 154.8345 86.4655) (width 0.25) (layer "F.Cu") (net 27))
 (segment (start 158.436045 77.156045) (end 158.436045 78.74) (width 0.25) (layer "F.Cu") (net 3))
 (segment (start 151.13 72.39) (end 152.4 73.66) (width 0.25) (layer "F.Cu") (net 3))
 (segment (start 151.13 70.01) (end 151.13 72.39) (width 0.25) (layer "F.Cu") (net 3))
 (segment (start 152.4 73.66) (end 154.94 73.66) (width 0.25) (layer "F.Cu") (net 3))
 (segment (start 154.94 73.66) (end 158.436045 77.156045) (width 0.25) (layer "F.Cu") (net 3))
 (segment (start 165.209378 76.309378) (end 165.209378 78.74) (width 0.25) (layer "F.Cu") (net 4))
 (segment (start 153.67 70.01) (end 153.67 71.753604) (width 0.25) (layer "F.Cu") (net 4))
 (segment (start 162.56 73.66) (end 165.209378 76.309378) (width 0.25) (layer "F.Cu") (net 4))
 (segment (start 153.67 71.753604) (end 155.576396 73.66) (width 0.25) (layer "F.Cu") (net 4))
 (segment (start 155.576396 73.66) (end 162.56 73.66) (width 0.25) (layer "F.Cu") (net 4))
 (segment (start 150.02 58.42) (end 147.32 58.42) (width 0.25) (layer "F.Cu") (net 16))
 (segment (start 147.32 73.66) (end 149.86 73.66) (width 0.25) (layer "F.Cu") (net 16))
 (segment (start 153.67 62.07) (end 150.02 58.42) (width 0.25) (layer "F.Cu") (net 16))
 (segment (start 147.32 58.42) (end 144.78 60.96) (width 0.25) (layer "F.Cu") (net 16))
 (segment (start 144.78 60.96) (end 144.78 71.12) (width 0.25) (layer "F.Cu") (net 16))
 (segment (start 144.78 71.12) (end 147.32 73.66) (width 0.25) (layer "F.Cu") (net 16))
 (segment (start 151.662712 75.462712) (end 151.662712 78.74) (width 0.25) (layer "F.Cu") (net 16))
 (segment (start 149.86 73.66) (end 151.662712 75.462712) (width 0.25) (layer "F.Cu") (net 16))
 (segment (start 185.42 38.1) (end 187.96 40.64) (width 0.25) (layer "B.Cu") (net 1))
 (segment (start 187.96 40.64) (end 187.96 66.04) (width 0.25) (layer "B.Cu") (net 1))
 (segment (start 177.8 76.6865) (end 177.8 73.66) (width 0.25) (layer "F.Cu") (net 19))
 (segment (start 185.42 84.3065) (end 177.8 76.6865) (width 0.25) (layer "F.Cu") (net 19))
 (segment (start 174.286666 84.3065) (end 185.42 84.3065) (width 0.25) (layer "B.Cu") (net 19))
 (segment (start 152.02 84.3065) (end 163.153333 84.3065) (width 0.25) (layer "B.Cu") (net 19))
 (segment (start 163.153333 84.3065) (end 174.286666 84.3065) (width 0.25) (layer "B.Cu") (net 19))
 (segment (start 185.1445 88.6245) (end 185.42 88.9) (width 0.25) (layer "F.Cu") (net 21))
 (segment (start 187.96 83.82) (end 182.88 78.74) (width 0.25) (layer "F.Cu") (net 21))
 (segment (start 174.286666 88.6245) (end 185.1445 88.6245) (width 0.25) (layer "F.Cu") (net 21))
 (segment (start 182.88 78.74) (end 182.88 73.66) (width 0.25) (layer "F.Cu") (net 21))
 (segment (start 185.6955 88.6245) (end 187.96 86.36) (width 0.25) (layer "F.Cu") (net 21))
 (segment (start 163.153333 88.6245) (end 174.286666 88.6245) (width 0.25) (layer "F.Cu") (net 21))
 (segment (start 152.02 88.6245) (end 163.153333 88.6245) (width 0.25) (layer "F.Cu") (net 21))
 (segment (start 185.42 88.6245) (end 185.6955 88.6245) (width 0.25) (layer "F.Cu") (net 21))
 (segment (start 187.96 86.36) (end 187.96 83.82) (width 0.25) (layer "F.Cu") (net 21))
 (segment (start 187.96 78.74) (end 190.5 81.28) (width 0.25) (layer "F.Cu") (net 2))
 (segment (start 190.5 88.9) (end 188.6165 90.7835) (width 0.25) (layer "F.Cu") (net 2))
 (segment (start 187.96 73.66) (end 187.96 78.74) (width 0.25) (layer "F.Cu") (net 2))
 (segment (start 190.5 81.28) (end 190.5 88.9) (width 0.25) (layer "F.Cu") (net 2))
 (segment (start 174.286666 90.7835) (end 163.153333 90.7835) (width 0.25) (layer "F.Cu") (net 2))
 (segment (start 188.6165 90.7835) (end 185.42 90.7835) (width 0.25) (layer "F.Cu") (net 2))
 (segment (start 174.286666 90.7835) (end 185.42 90.7835) (width 0.25) (layer "F.Cu") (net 2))
 (segment (start 152.02 90.7835) (end 163.153333 90.7835) (width 0.25) (layer "F.Cu") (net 2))
 (segment (start 159.706045 78.74) (end 159.706045 83.018212) (width 0.25) (layer "F.Cu") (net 18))
 (segment (start 159.706045 83.018212) (end 163.153333 86.4655) (width 0.25) (layer "F.Cu") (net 18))
 (segment (start 166.479378 80.119378) (end 167.64 81.28) (width 0.25) (layer "F.Cu") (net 20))
 (segment (start 170.2855 86.4655) (end 174.286666 86.4655) (width 0.25) (layer "F.Cu") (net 20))
 (segment (start 166.479378 78.74) (end 166.479378 80.119378) (width 0.25) (layer "F.Cu") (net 20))
 (segment (start 167.64 83.82) (end 170.2855 86.4655) (width 0.25) (layer "F.Cu") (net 20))
 (segment (start 167.64 81.28) (end 167.64 83.82) (width 0.25) (layer "F.Cu") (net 20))
 (segment (start 177.8 78.74) (end 180.34 81.28) (width 0.25) (layer "F.Cu") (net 17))
 (segment (start 173.252712 78.74) (end 177.8 78.74) (width 0.25) (layer "F.Cu") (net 17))
 (segment (start 180.34 81.28) (end 180.34 83.82) (width 0.25) (layer "F.Cu") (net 17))
 (segment (start 180.34 83.82) (end 182.9855 86.4655) (width 0.25) (layer "F.Cu") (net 17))
 (segment (start 182.9855 86.4655) (end 185.42 86.4655) (width 0.25) (layer "F.Cu") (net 17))
 (segment (start 169.73 73.21) (end 171.982712 75.462712) (width 0.25) (layer "F.Cu") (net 5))
 (segment (start 156.21 70.01) (end 159.41 73.21) (width 0.25) (layer "F.Cu") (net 5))
 (segment (start 159.41 73.21) (end 169.73 73.21) (width 0.25) (layer "F.Cu") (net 5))
 (segment (start 171.982712 75.462712) (end 171.982712 78.74) (width 0.25) (layer "F.Cu") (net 5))
 (segment (start 142.1 40.64) (end 147.32 35.42) (width 0.25) (layer "F.Cu") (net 24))
 (segment (start 135.668872 40.64) (end 142.1 40.64) (width 0.25) (layer "F.Cu") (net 24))
 (segment (start 157.48 33.02) (end 144.64 33.02) (width 0.25) (layer "F.Cu") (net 22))
 (segment (start 144.64 33.02) (end 142.24 35.42) (width 0.25) (layer "F.Cu") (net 22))
 (segment (start 160.02 35.56) (end 157.48 33.02) (width 0.25) (layer "F.Cu") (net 22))
 (segment (start 160.02 38.1) (end 160.02 35.56) (width 0.25) (layer "F.Cu") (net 22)))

